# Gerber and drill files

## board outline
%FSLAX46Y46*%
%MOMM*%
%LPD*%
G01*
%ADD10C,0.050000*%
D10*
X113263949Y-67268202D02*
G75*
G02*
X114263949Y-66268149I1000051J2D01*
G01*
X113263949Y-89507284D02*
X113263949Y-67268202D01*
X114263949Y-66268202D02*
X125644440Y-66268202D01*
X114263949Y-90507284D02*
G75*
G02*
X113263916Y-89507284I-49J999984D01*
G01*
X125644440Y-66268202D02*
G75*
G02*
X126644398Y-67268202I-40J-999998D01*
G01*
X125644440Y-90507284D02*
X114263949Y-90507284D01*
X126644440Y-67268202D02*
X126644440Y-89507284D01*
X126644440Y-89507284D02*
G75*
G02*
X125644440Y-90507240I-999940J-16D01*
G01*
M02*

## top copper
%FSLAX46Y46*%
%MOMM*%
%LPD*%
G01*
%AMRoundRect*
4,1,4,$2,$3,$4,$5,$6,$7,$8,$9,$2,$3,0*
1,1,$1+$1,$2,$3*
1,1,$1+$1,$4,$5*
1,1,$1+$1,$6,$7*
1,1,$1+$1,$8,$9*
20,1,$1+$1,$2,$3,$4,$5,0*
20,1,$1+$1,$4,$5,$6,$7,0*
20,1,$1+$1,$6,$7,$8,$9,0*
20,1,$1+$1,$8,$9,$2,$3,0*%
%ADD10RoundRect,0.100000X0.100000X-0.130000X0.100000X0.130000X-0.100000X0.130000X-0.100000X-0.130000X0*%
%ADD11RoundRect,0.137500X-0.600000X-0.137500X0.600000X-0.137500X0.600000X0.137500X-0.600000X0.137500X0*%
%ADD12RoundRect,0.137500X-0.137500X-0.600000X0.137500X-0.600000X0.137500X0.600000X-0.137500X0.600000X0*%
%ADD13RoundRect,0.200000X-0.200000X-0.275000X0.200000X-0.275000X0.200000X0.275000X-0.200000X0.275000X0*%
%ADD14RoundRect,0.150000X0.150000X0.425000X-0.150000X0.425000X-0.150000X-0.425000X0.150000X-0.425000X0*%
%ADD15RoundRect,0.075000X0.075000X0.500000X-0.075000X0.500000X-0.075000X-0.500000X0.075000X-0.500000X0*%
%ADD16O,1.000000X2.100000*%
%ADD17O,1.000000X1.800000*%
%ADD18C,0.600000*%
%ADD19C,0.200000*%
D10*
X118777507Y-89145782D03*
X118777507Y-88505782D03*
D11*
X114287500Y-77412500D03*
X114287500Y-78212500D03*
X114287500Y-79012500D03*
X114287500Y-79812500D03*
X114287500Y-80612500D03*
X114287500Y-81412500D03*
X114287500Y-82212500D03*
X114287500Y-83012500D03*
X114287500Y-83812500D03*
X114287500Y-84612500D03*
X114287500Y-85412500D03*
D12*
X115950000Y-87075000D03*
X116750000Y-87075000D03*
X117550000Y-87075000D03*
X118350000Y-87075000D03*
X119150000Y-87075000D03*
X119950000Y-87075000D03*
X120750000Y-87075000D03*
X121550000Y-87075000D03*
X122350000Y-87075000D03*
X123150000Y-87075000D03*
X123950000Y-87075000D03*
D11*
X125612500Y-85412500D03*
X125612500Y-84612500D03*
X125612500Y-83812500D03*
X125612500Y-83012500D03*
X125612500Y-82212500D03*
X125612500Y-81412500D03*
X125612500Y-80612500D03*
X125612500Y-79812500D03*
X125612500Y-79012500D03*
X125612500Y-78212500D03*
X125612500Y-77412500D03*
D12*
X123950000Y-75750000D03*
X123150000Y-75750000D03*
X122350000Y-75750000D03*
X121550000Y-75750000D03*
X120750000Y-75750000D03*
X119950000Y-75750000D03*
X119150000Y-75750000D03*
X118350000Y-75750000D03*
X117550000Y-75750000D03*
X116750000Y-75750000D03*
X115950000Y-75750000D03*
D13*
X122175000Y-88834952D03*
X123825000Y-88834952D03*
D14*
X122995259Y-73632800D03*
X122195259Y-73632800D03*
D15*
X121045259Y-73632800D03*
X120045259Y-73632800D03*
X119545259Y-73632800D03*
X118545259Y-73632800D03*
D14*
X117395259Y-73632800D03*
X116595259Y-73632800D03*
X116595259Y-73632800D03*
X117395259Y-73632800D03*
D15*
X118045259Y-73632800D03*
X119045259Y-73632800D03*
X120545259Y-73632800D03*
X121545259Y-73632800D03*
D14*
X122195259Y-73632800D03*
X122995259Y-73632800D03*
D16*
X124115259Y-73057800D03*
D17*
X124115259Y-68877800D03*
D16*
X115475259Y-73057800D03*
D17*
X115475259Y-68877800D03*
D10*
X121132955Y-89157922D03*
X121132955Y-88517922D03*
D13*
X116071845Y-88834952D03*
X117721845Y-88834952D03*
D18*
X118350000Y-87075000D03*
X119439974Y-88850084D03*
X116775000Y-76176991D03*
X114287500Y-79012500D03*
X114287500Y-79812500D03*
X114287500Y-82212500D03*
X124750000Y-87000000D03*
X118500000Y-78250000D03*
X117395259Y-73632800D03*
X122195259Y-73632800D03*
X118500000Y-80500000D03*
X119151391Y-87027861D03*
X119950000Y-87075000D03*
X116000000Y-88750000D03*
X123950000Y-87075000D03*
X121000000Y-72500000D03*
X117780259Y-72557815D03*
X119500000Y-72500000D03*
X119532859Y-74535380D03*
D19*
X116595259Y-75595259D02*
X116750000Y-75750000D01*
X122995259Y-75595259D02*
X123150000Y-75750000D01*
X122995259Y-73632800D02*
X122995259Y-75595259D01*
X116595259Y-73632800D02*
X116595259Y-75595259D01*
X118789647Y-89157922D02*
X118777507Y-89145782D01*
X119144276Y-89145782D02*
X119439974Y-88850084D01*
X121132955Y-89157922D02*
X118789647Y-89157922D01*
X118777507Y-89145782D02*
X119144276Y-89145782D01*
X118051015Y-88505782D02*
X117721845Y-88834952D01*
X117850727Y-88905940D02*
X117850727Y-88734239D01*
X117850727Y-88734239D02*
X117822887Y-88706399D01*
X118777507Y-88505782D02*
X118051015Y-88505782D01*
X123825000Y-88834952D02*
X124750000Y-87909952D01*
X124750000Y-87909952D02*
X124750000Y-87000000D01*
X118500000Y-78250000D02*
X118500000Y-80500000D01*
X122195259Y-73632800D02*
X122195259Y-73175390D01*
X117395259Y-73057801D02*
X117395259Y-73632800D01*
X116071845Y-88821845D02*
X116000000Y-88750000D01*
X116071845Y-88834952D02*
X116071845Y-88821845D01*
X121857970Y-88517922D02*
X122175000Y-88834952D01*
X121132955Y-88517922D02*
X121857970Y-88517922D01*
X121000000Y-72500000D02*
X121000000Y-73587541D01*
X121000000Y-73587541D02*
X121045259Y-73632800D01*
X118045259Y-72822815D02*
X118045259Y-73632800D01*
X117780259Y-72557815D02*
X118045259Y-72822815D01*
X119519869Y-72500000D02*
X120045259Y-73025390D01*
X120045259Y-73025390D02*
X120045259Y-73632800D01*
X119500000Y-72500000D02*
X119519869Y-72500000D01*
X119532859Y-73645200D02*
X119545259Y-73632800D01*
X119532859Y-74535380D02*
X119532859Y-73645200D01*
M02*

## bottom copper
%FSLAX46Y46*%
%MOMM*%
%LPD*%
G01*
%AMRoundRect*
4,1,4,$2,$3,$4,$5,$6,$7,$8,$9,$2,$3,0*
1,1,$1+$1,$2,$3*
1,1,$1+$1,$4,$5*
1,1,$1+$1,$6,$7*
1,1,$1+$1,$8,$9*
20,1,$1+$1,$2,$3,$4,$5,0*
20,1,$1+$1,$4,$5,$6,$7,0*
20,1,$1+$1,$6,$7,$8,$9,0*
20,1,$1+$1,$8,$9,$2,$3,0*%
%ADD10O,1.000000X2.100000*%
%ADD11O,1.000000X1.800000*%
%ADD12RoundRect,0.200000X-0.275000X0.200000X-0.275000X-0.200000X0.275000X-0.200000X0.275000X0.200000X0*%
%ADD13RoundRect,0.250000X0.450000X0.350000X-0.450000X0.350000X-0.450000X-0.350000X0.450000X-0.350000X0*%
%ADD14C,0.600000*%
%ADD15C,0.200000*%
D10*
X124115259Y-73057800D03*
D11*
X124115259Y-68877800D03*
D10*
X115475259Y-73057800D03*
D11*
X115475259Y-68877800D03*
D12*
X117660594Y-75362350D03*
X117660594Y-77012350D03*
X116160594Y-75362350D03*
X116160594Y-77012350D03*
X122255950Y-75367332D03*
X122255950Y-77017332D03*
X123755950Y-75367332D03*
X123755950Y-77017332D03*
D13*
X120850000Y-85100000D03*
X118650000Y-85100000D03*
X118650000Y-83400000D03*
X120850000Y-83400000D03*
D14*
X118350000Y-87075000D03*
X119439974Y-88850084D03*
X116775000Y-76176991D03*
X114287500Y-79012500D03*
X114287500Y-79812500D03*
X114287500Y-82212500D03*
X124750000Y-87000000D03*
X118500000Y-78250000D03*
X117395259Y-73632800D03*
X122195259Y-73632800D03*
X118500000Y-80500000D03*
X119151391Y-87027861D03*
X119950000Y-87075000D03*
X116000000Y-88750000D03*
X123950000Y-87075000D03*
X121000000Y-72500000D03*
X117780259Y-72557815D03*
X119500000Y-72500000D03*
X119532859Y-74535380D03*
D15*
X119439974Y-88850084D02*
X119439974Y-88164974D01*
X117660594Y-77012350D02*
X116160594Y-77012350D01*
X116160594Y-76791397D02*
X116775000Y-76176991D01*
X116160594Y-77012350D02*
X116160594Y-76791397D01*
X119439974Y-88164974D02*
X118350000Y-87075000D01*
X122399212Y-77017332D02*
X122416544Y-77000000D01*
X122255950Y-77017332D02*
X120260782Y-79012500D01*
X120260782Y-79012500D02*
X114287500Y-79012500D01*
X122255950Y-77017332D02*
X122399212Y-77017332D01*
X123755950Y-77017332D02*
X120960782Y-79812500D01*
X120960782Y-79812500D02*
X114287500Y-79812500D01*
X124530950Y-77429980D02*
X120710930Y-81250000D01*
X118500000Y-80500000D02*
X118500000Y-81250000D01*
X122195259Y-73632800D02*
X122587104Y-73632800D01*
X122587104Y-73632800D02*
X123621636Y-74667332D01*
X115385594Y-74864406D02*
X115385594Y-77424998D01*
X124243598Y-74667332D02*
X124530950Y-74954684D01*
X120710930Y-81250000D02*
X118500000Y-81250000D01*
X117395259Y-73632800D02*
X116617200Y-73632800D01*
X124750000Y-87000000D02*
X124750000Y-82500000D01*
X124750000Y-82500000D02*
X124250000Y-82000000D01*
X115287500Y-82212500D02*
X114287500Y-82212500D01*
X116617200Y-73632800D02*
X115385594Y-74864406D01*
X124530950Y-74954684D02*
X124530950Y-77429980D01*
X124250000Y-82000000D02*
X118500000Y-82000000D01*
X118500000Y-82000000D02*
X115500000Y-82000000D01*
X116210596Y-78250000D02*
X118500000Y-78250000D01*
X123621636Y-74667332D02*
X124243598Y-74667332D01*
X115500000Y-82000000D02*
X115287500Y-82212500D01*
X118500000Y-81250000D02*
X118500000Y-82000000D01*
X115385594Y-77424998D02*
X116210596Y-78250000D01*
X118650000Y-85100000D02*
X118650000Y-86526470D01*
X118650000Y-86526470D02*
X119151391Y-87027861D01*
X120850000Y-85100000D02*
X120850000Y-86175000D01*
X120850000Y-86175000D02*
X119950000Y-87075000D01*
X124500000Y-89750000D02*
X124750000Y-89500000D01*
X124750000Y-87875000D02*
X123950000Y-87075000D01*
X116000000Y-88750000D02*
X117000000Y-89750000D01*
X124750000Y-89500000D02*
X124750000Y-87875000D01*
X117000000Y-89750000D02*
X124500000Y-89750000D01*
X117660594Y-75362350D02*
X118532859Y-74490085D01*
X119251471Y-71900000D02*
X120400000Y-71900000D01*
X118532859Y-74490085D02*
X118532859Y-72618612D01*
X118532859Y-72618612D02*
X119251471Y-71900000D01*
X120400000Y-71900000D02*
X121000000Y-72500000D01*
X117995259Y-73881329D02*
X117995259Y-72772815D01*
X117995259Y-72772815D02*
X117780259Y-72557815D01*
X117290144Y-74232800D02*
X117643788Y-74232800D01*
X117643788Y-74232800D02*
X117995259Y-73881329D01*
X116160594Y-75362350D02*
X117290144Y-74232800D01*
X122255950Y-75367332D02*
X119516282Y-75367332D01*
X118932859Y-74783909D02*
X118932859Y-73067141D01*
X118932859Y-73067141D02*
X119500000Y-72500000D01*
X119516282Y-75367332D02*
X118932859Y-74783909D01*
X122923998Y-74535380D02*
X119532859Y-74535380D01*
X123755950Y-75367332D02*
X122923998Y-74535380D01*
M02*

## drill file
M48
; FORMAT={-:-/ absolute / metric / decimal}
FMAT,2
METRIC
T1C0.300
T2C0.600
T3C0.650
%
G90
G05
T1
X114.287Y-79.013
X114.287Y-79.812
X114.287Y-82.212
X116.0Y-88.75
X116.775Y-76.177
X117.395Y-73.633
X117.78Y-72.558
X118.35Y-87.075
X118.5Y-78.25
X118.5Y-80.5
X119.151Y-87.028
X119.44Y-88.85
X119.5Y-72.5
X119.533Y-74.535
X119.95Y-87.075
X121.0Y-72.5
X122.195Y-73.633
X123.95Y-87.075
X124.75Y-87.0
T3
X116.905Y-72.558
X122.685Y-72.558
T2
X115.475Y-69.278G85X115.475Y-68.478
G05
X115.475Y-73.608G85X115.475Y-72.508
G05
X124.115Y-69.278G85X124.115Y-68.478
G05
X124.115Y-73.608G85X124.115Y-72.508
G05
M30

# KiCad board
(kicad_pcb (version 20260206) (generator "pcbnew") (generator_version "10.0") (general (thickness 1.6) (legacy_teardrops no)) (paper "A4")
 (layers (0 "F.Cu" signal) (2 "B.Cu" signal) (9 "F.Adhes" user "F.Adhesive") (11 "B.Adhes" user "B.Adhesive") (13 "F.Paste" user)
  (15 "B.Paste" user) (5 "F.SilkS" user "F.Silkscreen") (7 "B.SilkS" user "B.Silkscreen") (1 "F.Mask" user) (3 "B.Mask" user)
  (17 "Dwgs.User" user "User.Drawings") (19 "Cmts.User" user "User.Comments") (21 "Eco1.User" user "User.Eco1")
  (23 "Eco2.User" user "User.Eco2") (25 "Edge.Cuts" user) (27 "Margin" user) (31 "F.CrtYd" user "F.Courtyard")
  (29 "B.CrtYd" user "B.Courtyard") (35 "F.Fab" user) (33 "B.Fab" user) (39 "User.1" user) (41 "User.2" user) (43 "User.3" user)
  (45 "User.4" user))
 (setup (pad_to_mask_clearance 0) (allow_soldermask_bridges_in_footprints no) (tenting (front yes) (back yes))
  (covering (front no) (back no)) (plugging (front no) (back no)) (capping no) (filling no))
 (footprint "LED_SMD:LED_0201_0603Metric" (layer "F.Cu") (at 118.777507 88.825782 90)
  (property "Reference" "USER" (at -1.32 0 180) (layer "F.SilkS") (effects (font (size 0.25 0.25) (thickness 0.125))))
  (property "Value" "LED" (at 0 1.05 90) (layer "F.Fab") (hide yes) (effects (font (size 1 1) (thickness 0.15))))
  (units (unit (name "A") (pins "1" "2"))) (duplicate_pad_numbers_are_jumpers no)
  (pad "" smd roundrect (at -0.345 0 90) (size 0.318 0.36) (layers "F.Paste") (roundrect_rratio 0.25))
  (pad "" smd roundrect (at 0.345 0 90) (size 0.318 0.36) (layers "F.Paste") (roundrect_rratio 0.25))
  (pad "1" smd roundrect (at -0.32 0 90) (size 0.46 0.4) (layers "F.Cu" "F.Mask") (roundrect_rratio 0.25) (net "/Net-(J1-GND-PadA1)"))
  (pad "2" smd roundrect (at 0.32 0 90) (size 0.46 0.4) (layers "F.Cu" "F.Mask") (roundrect_rratio 0.25) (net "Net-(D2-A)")))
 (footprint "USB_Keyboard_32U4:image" (layer "F.Cu") (at 114.351978 88.139877)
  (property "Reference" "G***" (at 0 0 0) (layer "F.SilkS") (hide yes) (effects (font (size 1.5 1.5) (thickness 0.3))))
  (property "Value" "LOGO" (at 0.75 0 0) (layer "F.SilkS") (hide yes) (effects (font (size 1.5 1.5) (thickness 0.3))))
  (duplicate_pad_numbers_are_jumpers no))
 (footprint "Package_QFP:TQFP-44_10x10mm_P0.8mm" (layer "F.Cu") (at 119.95 81.4125)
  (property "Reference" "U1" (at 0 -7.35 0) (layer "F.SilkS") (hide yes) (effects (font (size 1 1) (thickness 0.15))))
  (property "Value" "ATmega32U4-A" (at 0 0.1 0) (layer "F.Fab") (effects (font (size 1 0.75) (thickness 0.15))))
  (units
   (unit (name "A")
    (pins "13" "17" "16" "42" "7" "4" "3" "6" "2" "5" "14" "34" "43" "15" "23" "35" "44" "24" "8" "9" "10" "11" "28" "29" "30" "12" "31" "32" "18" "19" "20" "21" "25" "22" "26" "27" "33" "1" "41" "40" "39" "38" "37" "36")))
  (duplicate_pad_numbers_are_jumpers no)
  (pad "1" smd roundrect (at -5.6625 -4) (size 1.475 0.55) (layers "F.Cu" "F.Mask" "F.Paste") (roundrect_rratio 0.25)
   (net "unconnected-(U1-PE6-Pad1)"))
  (pad "2" smd roundrect (at -5.6625 -3.2) (size 1.475 0.55) (layers "F.Cu" "F.Mask" "F.Paste") (roundrect_rratio 0.25)
   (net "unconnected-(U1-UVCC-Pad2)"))
  (pad "3" smd roundrect (at -5.6625 -2.4) (size 1.475 0.55) (layers "F.Cu" "F.Mask" "F.Paste") (roundrect_rratio 0.25) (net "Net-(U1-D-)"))
  (pad "4" smd roundrect (at -5.6625 -1.6) (size 1.475 0.55) (layers "F.Cu" "F.Mask" "F.Paste") (roundrect_rratio 0.25) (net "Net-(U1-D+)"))
  (pad "5" smd roundrect (at -5.6625 -0.8) (size 1.475 0.55) (layers "F.Cu" "F.Mask" "F.Paste") (roundrect_rratio 0.25)
   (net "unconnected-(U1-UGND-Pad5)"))
  (pad "6" smd roundrect (at -5.6625 0) (size 1.475 0.55) (layers "F.Cu" "F.Mask" "F.Paste") (roundrect_rratio 0.25)
   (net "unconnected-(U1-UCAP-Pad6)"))
  (pad "7" smd roundrect (at -5.6625 0.8) (size 1.475 0.55) (layers "F.Cu" "F.Mask" "F.Paste") (roundrect_rratio 0.25) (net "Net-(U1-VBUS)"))
  (pad "8" smd roundrect (at -5.6625 1.6) (size 1.475 0.55) (layers "F.Cu" "F.Mask" "F.Paste") (roundrect_rratio 0.25)
   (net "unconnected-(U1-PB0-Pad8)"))
  (pad "9" smd roundrect (at -5.6625 2.4) (size 1.475 0.55) (layers "F.Cu" "F.Mask" "F.Paste") (roundrect_rratio 0.25)
   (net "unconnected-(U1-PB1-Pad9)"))
  (pad "10" smd roundrect (at -5.6625 3.2) (size 1.475 0.55) (layers "F.Cu" "F.Mask" "F.Paste") (roundrect_rratio 0.25)
   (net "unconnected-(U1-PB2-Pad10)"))
  (pad "11" smd roundrect (at -5.6625 4) (size 1.475 0.55) (layers "F.Cu" "F.Mask" "F.Paste") (roundrect_rratio 0.25)
   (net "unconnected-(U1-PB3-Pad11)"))
  (pad "12" smd roundrect (at -4 5.6625) (size 0.55 1.475) (layers "F.Cu" "F.Mask" "F.Paste") (roundrect_rratio 0.25)
   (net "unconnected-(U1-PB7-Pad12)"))
  (pad "13" smd roundrect (at -3.2 5.6625) (size 0.55 1.475) (layers "F.Cu" "F.Mask" "F.Paste") (roundrect_rratio 0.25)
   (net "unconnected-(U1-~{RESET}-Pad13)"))
  (pad "14" smd roundrect (at -2.4 5.6625) (size 0.55 1.475) (layers "F.Cu" "F.Mask" "F.Paste") (roundrect_rratio 0.25)
   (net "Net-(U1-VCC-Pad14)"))
  (pad "15" smd roundrect (at -1.6 5.6625) (size 0.55 1.475) (layers "F.Cu" "F.Mask" "F.Paste") (roundrect_rratio 0.25)
   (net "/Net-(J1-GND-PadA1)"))
  (pad "16" smd roundrect (at -0.8 5.6625) (size 0.55 1.475) (layers "F.Cu" "F.Mask" "F.Paste") (roundrect_rratio 0.25)
   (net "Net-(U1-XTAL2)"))
  (pad "17" smd roundrect (at 0 5.6625) (size 0.55 1.475) (layers "F.Cu" "F.Mask" "F.Paste") (roundrect_rratio 0.25) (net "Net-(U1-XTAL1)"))
  (pad "18" smd roundrect (at 0.8 5.6625) (size 0.55 1.475) (layers "F.Cu" "F.Mask" "F.Paste") (roundrect_rratio 0.25)
   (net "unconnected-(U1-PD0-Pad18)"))
  (pad "19" smd roundrect (at 1.6 5.6625) (size 0.55 1.475) (layers "F.Cu" "F.Mask" "F.Paste") (roundrect_rratio 0.25)
   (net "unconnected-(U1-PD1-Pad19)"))
  (pad "20" smd roundrect (at 2.4 5.6625) (size 0.55 1.475) (layers "F.Cu" "F.Mask" "F.Paste") (roundrect_rratio 0.25)
   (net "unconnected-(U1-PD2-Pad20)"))
  (pad "21" smd roundrect (at 3.2 5.6625) (size 0.55 1.475) (layers "F.Cu" "F.Mask" "F.Paste") (roundrect_rratio 0.25)
   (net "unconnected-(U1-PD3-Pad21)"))
  (pad "22" smd roundrect (at 4 5.6625) (size 0.55 1.475) (layers "F.Cu" "F.Mask" "F.Paste") (roundrect_rratio 0.25)
   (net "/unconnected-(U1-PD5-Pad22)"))
  (pad "23" smd roundrect (at 5.6625 4) (size 1.475 0.55) (layers "F.Cu" "F.Mask" "F.Paste") (roundrect_rratio 0.25)
   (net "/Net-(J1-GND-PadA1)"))
  (pad "24" smd roundrect (at 5.6625 3.2) (size 1.475 0.55) (layers "F.Cu" "F.Mask" "F.Paste") (roundrect_rratio 0.25)
   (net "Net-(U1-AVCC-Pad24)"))
  (pad "25" smd roundrect (at 5.6625 2.4) (size 1.475 0.55) (layers "F.Cu" "F.Mask" "F.Paste") (roundrect_rratio 0.25)
   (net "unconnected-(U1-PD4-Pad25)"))
  (pad "26" smd roundrect (at 5.6625 1.6) (size 1.475 0.55) (layers "F.Cu" "F.Mask" "F.Paste") (roundrect_rratio 0.25)
   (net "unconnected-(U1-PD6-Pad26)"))
  (pad "27" smd roundrect (at 5.6625 0.8) (size 1.475 0.55) (layers "F.Cu" "F.Mask" "F.Paste") (roundrect_rratio 0.25)
   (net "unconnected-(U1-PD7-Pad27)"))
  (pad "28" smd roundrect (at 5.6625 0) (size 1.475 0.55) (layers "F.Cu" "F.Mask" "F.Paste") (roundrect_rratio 0.25)
   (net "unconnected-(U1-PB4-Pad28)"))
  (pad "29" smd roundrect (at 5.6625 -0.8) (size 1.475 0.55) (layers "F.Cu" "F.Mask" "F.Paste") (roundrect_rratio 0.25)
   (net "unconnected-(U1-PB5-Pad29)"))
  (pad "30" smd roundrect (at 5.6625 -1.6) (size 1.475 0.55) (layers "F.Cu" "F.Mask" "F.Paste") (roundrect_rratio 0.25)
   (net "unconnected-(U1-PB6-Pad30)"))
  (pad "31" smd roundrect (at 5.6625 -2.4) (size 1.475 0.55) (layers "F.Cu" "F.Mask" "F.Paste") (roundrect_rratio 0.25)
   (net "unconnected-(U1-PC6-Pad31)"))
  (pad "32" smd roundrect (at 5.6625 -3.2) (size 1.475 0.55) (layers "F.Cu" "F.Mask" "F.Paste") (roundrect_rratio 0.25)
   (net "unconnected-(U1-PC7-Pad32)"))
  (pad "33" smd roundrect (at 5.6625 -4) (size 1.475 0.55) (layers "F.Cu" "F.Mask" "F.Paste") (roundrect_rratio 0.25)
   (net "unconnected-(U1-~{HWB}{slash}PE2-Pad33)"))
  (pad "34" smd roundrect (at 4 -5.6625) (size 0.55 1.475) (layers "F.Cu" "F.Mask" "F.Paste") (roundrect_rratio 0.25)
   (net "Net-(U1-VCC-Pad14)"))
  (pad "35" smd roundrect (at 3.2 -5.6625) (size 0.55 1.475) (layers "F.Cu" "F.Mask" "F.Paste") (roundrect_rratio 0.25)
   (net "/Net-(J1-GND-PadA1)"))
  (pad "36" smd roundrect (at 2.4 -5.6625) (size 0.55 1.475) (layers "F.Cu" "F.Mask" "F.Paste") (roundrect_rratio 0.25)
   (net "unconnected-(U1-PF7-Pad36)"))
  (pad "37" smd roundrect (at 1.6 -5.6625) (size 0.55 1.475) (layers "F.Cu" "F.Mask" "F.Paste") (roundrect_rratio 0.25)
   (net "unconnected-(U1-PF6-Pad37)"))
  (pad "38" smd roundrect (at 0.8 -5.6625) (size 0.55 1.475) (layers "F.Cu" "F.Mask" "F.Paste") (roundrect_rratio 0.25)
   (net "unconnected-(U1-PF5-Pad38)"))
  (pad "39" smd roundrect (at 0 -5.6625) (size 0.55 1.475) (layers "F.Cu" "F.Mask" "F.Paste") (roundrect_rratio 0.25)
   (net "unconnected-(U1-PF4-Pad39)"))
  (pad "40" smd roundrect (at -0.8 -5.6625) (size 0.55 1.475) (layers "F.Cu" "F.Mask" "F.Paste") (roundrect_rratio 0.25)
   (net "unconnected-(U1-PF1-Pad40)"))
  (pad "41" smd roundrect (at -1.6 -5.6625) (size 0.55 1.475) (layers "F.Cu" "F.Mask" "F.Paste") (roundrect_rratio 0.25)
   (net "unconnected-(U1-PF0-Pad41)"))
  (pad "42" smd roundrect (at -2.4 -5.6625) (size 0.55 1.475) (layers "F.Cu" "F.Mask" "F.Paste") (roundrect_rratio 0.25)
   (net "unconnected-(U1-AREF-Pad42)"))
  (pad "43" smd roundrect (at -3.2 -5.6625) (size 0.55 1.475) (layers "F.Cu" "F.Mask" "F.Paste") (roundrect_rratio 0.25)
   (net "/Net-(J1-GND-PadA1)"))
  (pad "44" smd roundrect (at -4 -5.6625) (size 0.55 1.475) (layers "F.Cu" "F.Mask" "F.Paste") (roundrect_rratio 0.25)
   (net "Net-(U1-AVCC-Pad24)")))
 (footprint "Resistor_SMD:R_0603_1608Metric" (layer "F.Cu") (at 123 88.834952)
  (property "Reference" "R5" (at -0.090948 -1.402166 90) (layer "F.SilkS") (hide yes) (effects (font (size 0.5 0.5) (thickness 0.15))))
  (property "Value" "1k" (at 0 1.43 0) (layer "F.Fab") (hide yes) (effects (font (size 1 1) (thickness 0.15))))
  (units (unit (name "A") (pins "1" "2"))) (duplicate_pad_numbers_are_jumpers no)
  (pad "1" smd roundrect (at -0.825 0) (size 0.8 0.95) (layers "F.Cu" "F.Mask" "F.Paste") (roundrect_rratio 0.25) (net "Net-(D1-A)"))
  (pad "2" smd roundrect (at 0.825 0) (size 0.8 0.95) (layers "F.Cu" "F.Mask" "F.Paste") (roundrect_rratio 0.25) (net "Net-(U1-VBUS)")))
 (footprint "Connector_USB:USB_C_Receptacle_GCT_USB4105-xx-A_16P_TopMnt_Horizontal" (layer "F.Cu") (at 119.795259 69.9528 180)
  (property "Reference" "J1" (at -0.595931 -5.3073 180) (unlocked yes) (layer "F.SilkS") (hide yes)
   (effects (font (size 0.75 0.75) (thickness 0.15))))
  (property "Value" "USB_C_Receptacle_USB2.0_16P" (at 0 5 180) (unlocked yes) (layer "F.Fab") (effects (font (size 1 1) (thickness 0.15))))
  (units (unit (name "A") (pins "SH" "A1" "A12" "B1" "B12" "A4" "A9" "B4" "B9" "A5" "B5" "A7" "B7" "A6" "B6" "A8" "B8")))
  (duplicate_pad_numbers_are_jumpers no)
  (pad "" np_thru_hole circle (at -2.89 -2.605 180) (size 0.65 0.65) (drill 0.65) (layers "*.Cu" "*.Mask"))
  (pad "" np_thru_hole circle (at 2.89 -2.605 180) (size 0.65 0.65) (drill 0.65) (layers "*.Cu" "*.Mask"))
  (pad "A1" smd roundrect (at -3.2 -3.68 180) (size 0.6 1.15) (layers "F.Cu" "F.Mask" "F.Paste") (roundrect_rratio 0.25)
   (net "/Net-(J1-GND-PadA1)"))
  (pad "A4" smd roundrect (at -2.4 -3.68 180) (size 0.6 1.15) (layers "F.Cu" "F.Mask" "F.Paste") (roundrect_rratio 0.25)
   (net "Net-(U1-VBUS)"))
  (pad "A5" smd roundrect (at -1.25 -3.68 180) (size 0.3 1.15) (layers "F.Cu" "F.Mask" "F.Paste") (roundrect_rratio 0.25)
   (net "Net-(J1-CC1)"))
  (pad "A6" smd roundrect (at -0.25 -3.68 180) (size 0.3 1.15) (layers "F.Cu" "F.Mask" "F.Paste") (roundrect_rratio 0.25)
   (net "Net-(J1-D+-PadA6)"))
  (pad "A7" smd roundrect (at 0.25 -3.68 180) (size 0.3 1.15) (layers "F.Cu" "F.Mask" "F.Paste") (roundrect_rratio 0.25)
   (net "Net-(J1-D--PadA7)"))
  (pad "A8" smd roundrect (at 1.25 -3.68 180) (size 0.3 1.15) (layers "F.Cu" "F.Mask" "F.Paste") (roundrect_rratio 0.25)
   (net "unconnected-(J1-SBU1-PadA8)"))
  (pad "A9" smd roundrect (at 2.4 -3.68 180) (size 0.6 1.15) (layers "F.Cu" "F.Mask" "F.Paste") (roundrect_rratio 0.25)
   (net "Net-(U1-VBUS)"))
  (pad "A12" smd roundrect (at 3.2 -3.68 180) (size 0.6 1.15) (layers "F.Cu" "F.Mask" "F.Paste") (roundrect_rratio 0.25)
   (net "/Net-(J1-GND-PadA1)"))
  (pad "B1" smd roundrect (at 3.2 -3.68 180) (size 0.6 1.15) (layers "F.Cu" "F.Mask" "F.Paste") (roundrect_rratio 0.25)
   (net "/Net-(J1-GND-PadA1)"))
  (pad "B4" smd roundrect (at 2.4 -3.68 180) (size 0.6 1.15) (layers "F.Cu" "F.Mask" "F.Paste") (roundrect_rratio 0.25)
   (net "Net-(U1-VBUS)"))
  (pad "B5" smd roundrect (at 1.75 -3.68 180) (size 0.3 1.15) (layers "F.Cu" "F.Mask" "F.Paste") (roundrect_rratio 0.25)
   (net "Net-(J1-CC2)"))
  (pad "B6" smd roundrect (at 0.75 -3.68 180) (size 0.3 1.15) (layers "F.Cu" "F.Mask" "F.Paste") (roundrect_rratio 0.25)
   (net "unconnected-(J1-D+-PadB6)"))
  (pad "B7" smd roundrect (at -0.75 -3.68 180) (size 0.3 1.15) (layers "F.Cu" "F.Mask" "F.Paste") (roundrect_rratio 0.25)
   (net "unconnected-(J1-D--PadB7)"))
  (pad "B8" smd roundrect (at -1.75 -3.68 180) (size 0.3 1.15) (layers "F.Cu" "F.Mask" "F.Paste") (roundrect_rratio 0.25)
   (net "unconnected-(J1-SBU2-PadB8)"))
  (pad "B9" smd roundrect (at -2.4 -3.68 180) (size 0.6 1.15) (layers "F.Cu" "F.Mask" "F.Paste") (roundrect_rratio 0.25)
   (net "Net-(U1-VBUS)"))
  (pad "B12" smd roundrect (at -3.2 -3.68 180) (size 0.6 1.15) (layers "F.Cu" "F.Mask" "F.Paste") (roundrect_rratio 0.25)
   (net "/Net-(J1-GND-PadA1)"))
  (pad "SH" thru_hole oval (at -4.32 -3.105 180) (size 1 2.1) (drill oval 0.6 1.7) (layers "*.Cu" "*.Mask" "F.Paste")
   (remove_unused_layers no) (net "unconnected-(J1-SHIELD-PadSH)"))
  (pad "SH" thru_hole oval (at -4.32 1.075 180) (size 1 1.8) (drill oval 0.6 1.4) (layers "*.Cu" "*.Mask" "F.Paste")
   (remove_unused_layers no) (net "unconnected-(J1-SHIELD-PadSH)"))
  (pad "SH" thru_hole oval (at 4.32 -3.105 180) (size 1 2.1) (drill oval 0.6 1.7) (layers "*.Cu" "*.Mask" "F.Paste")
   (remove_unused_layers no) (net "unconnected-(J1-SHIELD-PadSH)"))
  (pad "SH" thru_hole oval (at 4.32 1.075 180) (size 1 1.8) (drill oval 0.6 1.4) (layers "*.Cu" "*.Mask" "F.Paste")
   (remove_unused_layers no) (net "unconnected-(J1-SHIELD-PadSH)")))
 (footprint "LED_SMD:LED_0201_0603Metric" (layer "F.Cu") (at 121.132955 88.837922 90)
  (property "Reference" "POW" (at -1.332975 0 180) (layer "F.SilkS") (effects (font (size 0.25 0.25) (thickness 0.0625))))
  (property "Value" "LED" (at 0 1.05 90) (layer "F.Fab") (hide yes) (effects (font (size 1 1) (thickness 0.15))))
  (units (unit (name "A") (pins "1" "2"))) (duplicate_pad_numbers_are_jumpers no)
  (pad "" smd roundrect (at -0.345 0 90) (size 0.318 0.36) (layers "F.Paste") (roundrect_rratio 0.25))
  (pad "" smd roundrect (at 0.345 0 90) (size 0.318 0.36) (layers "F.Paste") (roundrect_rratio 0.25))
  (pad "1" smd roundrect (at -0.32 0 90) (size 0.46 0.4) (layers "F.Cu" "F.Mask") (roundrect_rratio 0.25) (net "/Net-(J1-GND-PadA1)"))
  (pad "2" smd roundrect (at 0.32 0 90) (size 0.46 0.4) (layers "F.Cu" "F.Mask") (roundrect_rratio 0.25) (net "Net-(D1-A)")))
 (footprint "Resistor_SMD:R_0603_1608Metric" (layer "F.Cu") (at 116.896845 88.834952)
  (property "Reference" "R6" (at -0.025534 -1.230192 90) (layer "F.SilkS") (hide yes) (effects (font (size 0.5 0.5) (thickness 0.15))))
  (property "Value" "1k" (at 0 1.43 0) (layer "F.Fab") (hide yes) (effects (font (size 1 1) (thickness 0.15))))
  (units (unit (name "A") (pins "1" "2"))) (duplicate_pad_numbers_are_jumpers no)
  (pad "1" smd roundrect (at -0.825 0) (size 0.8 0.95) (layers "F.Cu" "F.Mask" "F.Paste") (roundrect_rratio 0.25)
   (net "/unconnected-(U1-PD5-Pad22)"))
  (pad "2" smd roundrect (at 0.825 0) (size 0.8 0.95) (layers "F.Cu" "F.Mask" "F.Paste") (roundrect_rratio 0.25) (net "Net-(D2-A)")))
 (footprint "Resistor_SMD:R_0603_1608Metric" (layer "B.Cu") (at 117.660594 76.18735 -90)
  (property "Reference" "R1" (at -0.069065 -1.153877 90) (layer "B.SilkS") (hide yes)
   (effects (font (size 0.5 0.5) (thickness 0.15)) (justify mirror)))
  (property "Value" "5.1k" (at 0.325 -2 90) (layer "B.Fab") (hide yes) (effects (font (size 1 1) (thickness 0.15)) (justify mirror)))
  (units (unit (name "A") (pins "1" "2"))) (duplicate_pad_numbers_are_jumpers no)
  (pad "1" smd roundrect (at -0.825 0 270) (size 0.8 0.95) (layers "B.Cu" "B.Mask" "B.Paste") (roundrect_rratio 0.25) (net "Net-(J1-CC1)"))
  (pad "2" smd roundrect (at 0.825 0 270) (size 0.8 0.95) (layers "B.Cu" "B.Mask" "B.Paste") (roundrect_rratio 0.25)
   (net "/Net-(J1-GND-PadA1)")))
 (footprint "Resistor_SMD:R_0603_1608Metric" (layer "B.Cu") (at 116.160594 76.18735 -90)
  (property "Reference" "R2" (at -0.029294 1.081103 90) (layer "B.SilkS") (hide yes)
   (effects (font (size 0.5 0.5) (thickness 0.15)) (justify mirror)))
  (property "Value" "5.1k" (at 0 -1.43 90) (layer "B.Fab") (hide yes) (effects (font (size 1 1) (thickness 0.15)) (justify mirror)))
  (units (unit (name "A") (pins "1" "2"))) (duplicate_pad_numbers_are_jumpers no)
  (pad "1" smd roundrect (at -0.825 0 270) (size 0.8 0.95) (layers "B.Cu" "B.Mask" "B.Paste") (roundrect_rratio 0.25) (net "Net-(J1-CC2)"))
  (pad "2" smd roundrect (at 0.825 0 270) (size 0.8 0.95) (layers "B.Cu" "B.Mask" "B.Paste") (roundrect_rratio 0.25)
   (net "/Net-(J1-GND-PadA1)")))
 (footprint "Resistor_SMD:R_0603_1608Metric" (layer "B.Cu") (at 122.25595 76.192332 -90)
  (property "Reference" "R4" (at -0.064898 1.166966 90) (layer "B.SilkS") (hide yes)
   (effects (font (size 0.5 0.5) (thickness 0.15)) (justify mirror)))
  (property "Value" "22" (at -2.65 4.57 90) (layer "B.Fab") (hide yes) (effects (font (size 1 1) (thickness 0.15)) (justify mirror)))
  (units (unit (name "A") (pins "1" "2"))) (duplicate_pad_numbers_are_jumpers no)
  (pad "1" smd roundrect (at -0.825 0 270) (size 0.8 0.95) (layers "B.Cu" "B.Mask" "B.Paste") (roundrect_rratio 0.25)
   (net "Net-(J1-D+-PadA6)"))
  (pad "2" smd roundrect (at 0.825 0 270) (size 0.8 0.95) (layers "B.Cu" "B.Mask" "B.Paste") (roundrect_rratio 0.25) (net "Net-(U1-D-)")))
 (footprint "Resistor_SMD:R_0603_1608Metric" (layer "B.Cu") (at 123.75595 76.192332 -90)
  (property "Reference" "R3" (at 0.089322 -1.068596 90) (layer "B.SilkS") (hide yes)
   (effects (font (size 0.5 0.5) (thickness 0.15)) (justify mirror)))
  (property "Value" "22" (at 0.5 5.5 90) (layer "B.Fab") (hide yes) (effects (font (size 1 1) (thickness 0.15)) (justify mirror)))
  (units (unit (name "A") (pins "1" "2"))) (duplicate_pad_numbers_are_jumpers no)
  (pad "1" smd roundrect (at -0.825 0 270) (size 0.8 0.95) (layers "B.Cu" "B.Mask" "B.Paste") (roundrect_rratio 0.25)
   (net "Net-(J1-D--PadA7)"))
  (pad "2" smd roundrect (at 0.825 0 270) (size 0.8 0.95) (layers "B.Cu" "B.Mask" "B.Paste") (roundrect_rratio 0.25) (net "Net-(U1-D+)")))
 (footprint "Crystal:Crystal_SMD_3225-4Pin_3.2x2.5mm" (layer "B.Cu") (at 119.75 84.25 180)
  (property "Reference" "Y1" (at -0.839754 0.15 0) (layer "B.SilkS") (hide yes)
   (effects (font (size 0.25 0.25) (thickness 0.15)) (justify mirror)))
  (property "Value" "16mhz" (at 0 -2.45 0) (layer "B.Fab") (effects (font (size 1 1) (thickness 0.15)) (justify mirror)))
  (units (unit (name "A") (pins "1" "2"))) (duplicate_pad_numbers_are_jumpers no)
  (pad "1" smd roundrect (at -1.1 -0.85 180) (size 1.4 1.2) (layers "B.Cu" "B.Mask" "B.Paste") (roundrect_rratio 0.208333)
   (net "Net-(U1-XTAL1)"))
  (pad "2" smd roundrect (at 1.1 -0.85 180) (size 1.4 1.2) (layers "B.Cu" "B.Mask" "B.Paste") (roundrect_rratio 0.208333)
   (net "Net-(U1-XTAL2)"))
  (pad "3" smd roundrect (at 1.1 0.85 180) (size 1.4 1.2) (layers "B.Cu" "B.Mask" "B.Paste") (roundrect_rratio 0.208333))
  (pad "4" smd roundrect (at -1.1 0.85 180) (size 1.4 1.2) (layers "B.Cu" "B.Mask" "B.Paste") (roundrect_rratio 0.208333)))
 (gr_arc (start 113.263949 67.268202) (mid 113.556844 66.561111) (end 114.263949 66.268202) (stroke (width 0.05) (type default))
  (layer "Edge.Cuts"))
 (gr_line (start 113.263949 89.507284) (end 113.263949 67.268202) (stroke (width 0.05) (type default)) (layer "Edge.Cuts"))
 (gr_line (start 114.263949 66.268202) (end 125.64444 66.268202) (stroke (width 0.05) (type default)) (layer "Edge.Cuts"))
 (gr_arc (start 114.263949 90.507284) (mid 113.556842 90.214391) (end 113.263949 89.507284) (stroke (width 0.05) (type default))
  (layer "Edge.Cuts"))
 (gr_arc (start 125.64444 66.268202) (mid 126.351547 66.561095) (end 126.64444 67.268202) (stroke (width 0.05) (type default))
  (layer "Edge.Cuts"))
 (gr_line (start 125.64444 90.507284) (end 114.263949 90.507284) (stroke (width 0.05) (type default)) (layer "Edge.Cuts"))
 (gr_line (start 126.64444 67.268202) (end 126.64444 89.507284) (stroke (width 0.05) (type default)) (layer "Edge.Cuts"))
 (gr_arc (start 126.64444 89.507284) (mid 126.351555 90.214415) (end 125.64444 90.507284) (stroke (width 0.05) (type default))
  (layer "Edge.Cuts"))
 (segment (start 116.595259 75.595259) (end 116.75 75.75) (width 0.2) (layer "F.Cu") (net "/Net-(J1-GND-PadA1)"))
 (segment (start 122.995259 75.595259) (end 123.15 75.75) (width 0.2) (layer "F.Cu") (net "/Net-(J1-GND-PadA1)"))
 (segment (start 122.995259 73.6328) (end 122.995259 75.595259) (width 0.2) (layer "F.Cu") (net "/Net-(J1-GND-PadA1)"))
 (segment (start 116.595259 73.6328) (end 116.595259 75.595259) (width 0.2) (layer "F.Cu") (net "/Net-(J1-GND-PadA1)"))
 (segment (start 118.789647 89.157922) (end 118.777507 89.145782) (width 0.2) (layer "F.Cu") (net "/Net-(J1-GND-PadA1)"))
 (segment (start 119.144276 89.145782) (end 119.439974 88.850084) (width 0.2) (layer "F.Cu") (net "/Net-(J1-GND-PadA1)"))
 (segment (start 121.132955 89.157922) (end 118.789647 89.157922) (width 0.2) (layer "F.Cu") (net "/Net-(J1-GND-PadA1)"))
 (segment (start 118.777507 89.145782) (end 119.144276 89.145782) (width 0.2) (layer "F.Cu") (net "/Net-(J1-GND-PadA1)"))
 (via (at 118.35 87.075) (size 0.6) (drill 0.3) (layers "F.Cu" "B.Cu") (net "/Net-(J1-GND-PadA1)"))
 (via (at 119.439974 88.850084) (size 0.6) (drill 0.3) (layers "F.Cu" "B.Cu") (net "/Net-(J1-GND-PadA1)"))
 (via (at 116.775 76.176991) (size 0.6) (drill 0.3) (layers "F.Cu" "B.Cu") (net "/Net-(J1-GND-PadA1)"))
 (segment (start 119.439974 88.850084) (end 119.439974 88.164974) (width 0.2) (layer "B.Cu") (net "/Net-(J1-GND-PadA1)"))
 (segment (start 117.660594 77.01235) (end 116.160594 77.01235) (width 0.2) (layer "B.Cu") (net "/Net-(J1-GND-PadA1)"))
 (segment (start 116.160594 76.791397) (end 116.775 76.176991) (width 0.2) (layer "B.Cu") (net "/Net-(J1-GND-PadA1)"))
 (segment (start 116.160594 77.01235) (end 116.160594 76.791397) (width 0.2) (layer "B.Cu") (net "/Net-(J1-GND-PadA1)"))
 (segment (start 119.439974 88.164974) (end 118.35 87.075) (width 0.2) (layer "B.Cu") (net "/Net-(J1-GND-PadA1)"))
 (segment (start 118.051015 88.505782) (end 117.721845 88.834952) (width 0.2) (layer "F.Cu") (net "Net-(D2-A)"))
 (segment (start 117.850727 88.90594) (end 117.850727 88.734239) (width 0.2) (layer "F.Cu") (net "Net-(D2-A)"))
 (segment (start 117.850727 88.734239) (end 117.822887 88.706399) (width 0.2) (layer "F.Cu") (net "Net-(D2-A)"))
 (segment (start 118.777507 88.505782) (end 118.051015 88.505782) (width 0.2) (layer "F.Cu") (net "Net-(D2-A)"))
 (via (at 114.2875 79.0125) (size 0.6) (drill 0.3) (layers "F.Cu" "B.Cu") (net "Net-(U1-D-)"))
 (segment (start 122.399212 77.017332) (end 122.416544 77) (width 0.2) (layer "B.Cu") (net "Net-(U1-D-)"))
 (segment (start 122.25595 77.017332) (end 120.260782 79.0125) (width 0.2) (layer "B.Cu") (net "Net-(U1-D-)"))
 (segment (start 120.260782 79.0125) (end 114.2875 79.0125) (width 0.2) (layer "B.Cu") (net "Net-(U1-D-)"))
 (segment (start 122.25595 77.017332) (end 122.399212 77.017332) (width 0.2) (layer "B.Cu") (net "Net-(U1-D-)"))
 (via (at 114.2875 79.8125) (size 0.6) (drill 0.3) (layers "F.Cu" "B.Cu") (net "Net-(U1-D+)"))
 (segment (start 123.75595 77.017332) (end 120.960782 79.8125) (width 0.2) (layer "B.Cu") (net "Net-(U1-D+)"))
 (segment (start 120.960782 79.8125) (end 114.2875 79.8125) (width 0.2) (layer "B.Cu") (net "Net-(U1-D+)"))
 (segment (start 123.825 88.834952) (end 124.75 87.909952) (width 0.2) (layer "F.Cu") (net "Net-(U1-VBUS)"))
 (segment (start 124.75 87.909952) (end 124.75 87) (width 0.2) (layer "F.Cu") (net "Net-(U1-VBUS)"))
 (segment (start 118.5 78.25) (end 118.5 80.5) (width 0.2) (layer "F.Cu") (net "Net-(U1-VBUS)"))
 (segment (start 122.195259 73.6328) (end 122.195259 73.17539) (width 0.2) (layer "F.Cu") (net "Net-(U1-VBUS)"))
 (segment (start 117.395259 73.057801) (end 117.395259 73.6328) (width 0.2) (layer "F.Cu") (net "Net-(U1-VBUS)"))
 (via (at 114.2875 82.2125) (size 0.6) (drill 0.3) (layers "F.Cu" "B.Cu") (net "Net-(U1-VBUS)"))
 (via (at 124.75 87) (size 0.6) (drill 0.3) (layers "F.Cu" "B.Cu") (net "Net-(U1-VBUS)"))
 (via (at 118.5 78.25) (size 0.6) (drill 0.3) (layers "F.Cu" "B.Cu") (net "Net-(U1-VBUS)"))
 (via (at 117.395259 73.6328) (size 0.6) (drill 0.3) (layers "F.Cu" "B.Cu") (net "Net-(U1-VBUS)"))
 (via (at 122.195259 73.6328) (size 0.6) (drill 0.3) (layers "F.Cu" "B.Cu") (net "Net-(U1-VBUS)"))
 (via (at 118.5 80.5) (size 0.6) (drill 0.3) (layers "F.Cu" "B.Cu") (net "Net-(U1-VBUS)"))
 (segment (start 124.53095 77.42998) (end 120.71093 81.25) (width 0.2) (layer "B.Cu") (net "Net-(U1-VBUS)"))
 (segment (start 118.5 80.5) (end 118.5 81.25) (width 0.2) (layer "B.Cu") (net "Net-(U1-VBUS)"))
 (segment (start 122.195259 73.6328) (end 122.587104 73.6328) (width 0.2) (layer "B.Cu") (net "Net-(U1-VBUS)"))
 (segment (start 122.587104 73.6328) (end 123.621636 74.667332) (width 0.2) (layer "B.Cu") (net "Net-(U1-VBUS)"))
 (segment (start 115.385594 74.864406) (end 115.385594 77.424998) (width 0.2) (layer "B.Cu") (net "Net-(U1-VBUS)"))
 (segment (start 124.243598 74.667332) (end 124.53095 74.954684) (width 0.2) (layer "B.Cu") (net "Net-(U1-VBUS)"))
 (segment (start 120.71093 81.25) (end 118.5 81.25) (width 0.2) (layer "B.Cu") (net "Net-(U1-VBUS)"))
 (segment (start 117.395259 73.6328) (end 116.6172 73.6328) (width 0.2) (layer "B.Cu") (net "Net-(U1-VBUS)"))
 (segment (start 124.75 87) (end 124.75 82.5) (width 0.2) (layer "B.Cu") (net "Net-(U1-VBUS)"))
 (segment (start 124.75 82.5) (end 124.25 82) (width 0.2) (layer "B.Cu") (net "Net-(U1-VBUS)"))
 (segment (start 115.2875 82.2125) (end 114.2875 82.2125) (width 0.2) (layer "B.Cu") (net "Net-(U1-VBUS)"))
 (segment (start 116.6172 73.6328) (end 115.385594 74.864406) (width 0.2) (layer "B.Cu") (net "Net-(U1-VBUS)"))
 (segment (start 124.53095 74.954684) (end 124.53095 77.42998) (width 0.2) (layer "B.Cu") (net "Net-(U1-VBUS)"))
 (segment (start 124.25 82) (end 118.5 82) (width 0.2) (layer "B.Cu") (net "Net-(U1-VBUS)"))
 (segment (start 118.5 82) (end 115.5 82) (width 0.2) (layer "B.Cu") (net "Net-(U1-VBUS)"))
 (segment (start 116.210596 78.25) (end 118.5 78.25) (width 0.2) (layer "B.Cu") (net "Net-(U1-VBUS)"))
 (segment (start 123.621636 74.667332) (end 124.243598 74.667332) (width 0.2) (layer "B.Cu") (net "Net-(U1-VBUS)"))
 (segment (start 115.5 82) (end 115.2875 82.2125) (width 0.2) (layer "B.Cu") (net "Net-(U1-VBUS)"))
 (segment (start 118.5 81.25) (end 118.5 82) (width 0.2) (layer "B.Cu") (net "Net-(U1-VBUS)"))
 (segment (start 115.385594 77.424998) (end 116.210596 78.25) (width 0.2) (layer "B.Cu") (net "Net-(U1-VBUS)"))
 (via (at 119.151391 87.027861) (size 0.6) (drill 0.3) (layers "F.Cu" "B.Cu") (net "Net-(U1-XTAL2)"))
 (segment (start 118.65 85.1) (end 118.65 86.52647) (width 0.2) (layer "B.Cu") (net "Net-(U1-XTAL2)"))
 (segment (start 118.65 86.52647) (end 119.151391 87.027861) (width 0.2) (layer "B.Cu") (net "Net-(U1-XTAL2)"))
 (via (at 119.95 87.075) (size 0.6) (drill 0.3) (layers "F.Cu" "B.Cu") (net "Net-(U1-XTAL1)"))
 (segment (start 120.85 85.1) (end 120.85 86.175) (width 0.2) (layer "B.Cu") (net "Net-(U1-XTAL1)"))
 (segment (start 120.85 86.175) (end 119.95 87.075) (width 0.2) (layer "B.Cu") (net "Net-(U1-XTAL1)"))
 (segment (start 116.071845 88.821845) (end 116 88.75) (width 0.2) (layer "F.Cu") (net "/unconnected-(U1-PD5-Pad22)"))
 (segment (start 116.071845 88.834952) (end 116.071845 88.821845) (width 0.2) (layer "F.Cu") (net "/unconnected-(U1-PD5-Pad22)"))
 (via (at 116 88.75) (size 0.6) (drill 0.3) (layers "F.Cu" "B.Cu") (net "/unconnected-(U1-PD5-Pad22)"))
 (via (at 123.95 87.075) (size 0.6) (drill 0.3) (layers "F.Cu" "B.Cu") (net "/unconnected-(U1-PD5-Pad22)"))
 (segment (start 124.5 89.75) (end 124.75 89.5) (width 0.2) (layer "B.Cu") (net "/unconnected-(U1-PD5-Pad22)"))
 (segment (start 124.75 87.875) (end 123.95 87.075) (width 0.2) (layer "B.Cu") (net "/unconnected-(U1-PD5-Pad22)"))
 (segment (start 116 88.75) (end 117 89.75) (width 0.2) (layer "B.Cu") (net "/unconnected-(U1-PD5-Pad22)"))
 (segment (start 124.75 89.5) (end 124.75 87.875) (width 0.2) (layer "B.Cu") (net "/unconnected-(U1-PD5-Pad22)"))
 (segment (start 117 89.75) (end 124.5 89.75) (width 0.2) (layer "B.Cu") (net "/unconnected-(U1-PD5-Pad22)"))
 (segment (start 121.85797 88.517922) (end 122.175 88.834952) (width 0.2) (layer "F.Cu") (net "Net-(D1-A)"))
 (segment (start 121.132955 88.517922) (end 121.85797 88.517922) (width 0.2) (layer "F.Cu") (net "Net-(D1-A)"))
 (segment (start 121 72.5) (end 121 73.587541) (width 0.2) (layer "F.Cu") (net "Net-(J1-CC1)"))
 (segment (start 121 73.587541) (end 121.045259 73.6328) (width 0.2) (layer "F.Cu") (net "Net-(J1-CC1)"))
 (via (at 121 72.5) (size 0.6) (drill 0.3) (layers "F.Cu" "B.Cu") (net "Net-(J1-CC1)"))
 (segment (start 117.660594 75.36235) (end 118.532859 74.490085) (width 0.2) (layer "B.Cu") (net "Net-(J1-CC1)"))
 (segment (start 119.251471 71.9) (end 120.4 71.9) (width 0.2) (layer "B.Cu") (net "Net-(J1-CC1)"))
 (segment (start 118.532859 74.490085) (end 118.532859 72.618612) (width 0.2) (layer "B.Cu") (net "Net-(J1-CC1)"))
 (segment (start 118.532859 72.618612) (end 119.251471 71.9) (width 0.2) (layer "B.Cu") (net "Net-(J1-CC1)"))
 (segment (start 120.4 71.9) (end 121 72.5) (width 0.2) (layer "B.Cu") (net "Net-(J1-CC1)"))
 (segment (start 118.045259 72.822815) (end 118.045259 73.6328) (width 0.2) (layer "F.Cu") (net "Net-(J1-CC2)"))
 (segment (start 117.780259 72.557815) (end 118.045259 72.822815) (width 0.2) (layer "F.Cu") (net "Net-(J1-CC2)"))
 (via (at 117.780259 72.557815) (size 0.6) (drill 0.3) (layers "F.Cu" "B.Cu") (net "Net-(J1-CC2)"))
 (segment (start 117.995259 73.881329) (end 117.995259 72.772815) (width 0.2) (layer "B.Cu") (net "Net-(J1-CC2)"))
 (segment (start 117.995259 72.772815) (end 117.780259 72.557815) (width 0.2) (layer "B.Cu") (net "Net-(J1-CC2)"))
 (segment (start 117.290144 74.2328) (end 117.643788 74.2328) (width 0.2) (layer "B.Cu") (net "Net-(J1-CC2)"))
 (segment (start 117.643788 74.2328) (end 117.995259 73.881329) (width 0.2) (layer "B.Cu") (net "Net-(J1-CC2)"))
 (segment (start 116.160594 75.36235) (end 117.290144 74.2328) (width 0.2) (layer "B.Cu") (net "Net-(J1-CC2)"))
 (segment (start 119.519869 72.5) (end 120.045259 73.02539) (width 0.2) (layer "F.Cu") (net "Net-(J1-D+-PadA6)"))
 (segment (start 120.045259 73.02539) (end 120.045259 73.6328) (width 0.2) (layer "F.Cu") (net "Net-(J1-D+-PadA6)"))
 (segment (start 119.5 72.5) (end 119.519869 72.5) (width 0.2) (layer "F.Cu") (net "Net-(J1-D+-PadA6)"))
 (via (at 119.5 72.5) (size 0.6) (drill 0.3) (layers "F.Cu" "B.Cu") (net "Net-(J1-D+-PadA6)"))
 (segment (start 122.25595 75.367332) (end 119.516282 75.367332) (width 0.2) (layer "B.Cu") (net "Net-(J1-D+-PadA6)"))
 (segment (start 118.932859 74.783909) (end 118.932859 73.067141) (width 0.2) (layer "B.Cu") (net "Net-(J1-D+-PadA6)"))
 (segment (start 118.932859 73.067141) (end 119.5 72.5) (width 0.2) (layer "B.Cu") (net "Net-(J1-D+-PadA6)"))
 (segment (start 119.516282 75.367332) (end 118.932859 74.783909) (width 0.2) (layer "B.Cu") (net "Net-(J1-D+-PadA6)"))
 (segment (start 119.532859 73.6452) (end 119.545259 73.6328) (width 0.2) (layer "F.Cu") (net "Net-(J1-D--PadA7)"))
 (segment (start 119.532859 74.53538) (end 119.532859 73.6452) (width 0.2) (layer "F.Cu") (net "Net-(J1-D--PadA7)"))
 (via (at 119.532859 74.53538) (size 0.6) (drill 0.3) (layers "F.Cu" "B.Cu") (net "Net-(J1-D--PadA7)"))
 (segment (start 122.923998 74.53538) (end 119.532859 74.53538) (width 0.2) (layer "B.Cu") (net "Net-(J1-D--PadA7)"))
 (segment (start 123.75595 75.367332) (end 122.923998 74.53538) (width 0.2) (layer "B.Cu") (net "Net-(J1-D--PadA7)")))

